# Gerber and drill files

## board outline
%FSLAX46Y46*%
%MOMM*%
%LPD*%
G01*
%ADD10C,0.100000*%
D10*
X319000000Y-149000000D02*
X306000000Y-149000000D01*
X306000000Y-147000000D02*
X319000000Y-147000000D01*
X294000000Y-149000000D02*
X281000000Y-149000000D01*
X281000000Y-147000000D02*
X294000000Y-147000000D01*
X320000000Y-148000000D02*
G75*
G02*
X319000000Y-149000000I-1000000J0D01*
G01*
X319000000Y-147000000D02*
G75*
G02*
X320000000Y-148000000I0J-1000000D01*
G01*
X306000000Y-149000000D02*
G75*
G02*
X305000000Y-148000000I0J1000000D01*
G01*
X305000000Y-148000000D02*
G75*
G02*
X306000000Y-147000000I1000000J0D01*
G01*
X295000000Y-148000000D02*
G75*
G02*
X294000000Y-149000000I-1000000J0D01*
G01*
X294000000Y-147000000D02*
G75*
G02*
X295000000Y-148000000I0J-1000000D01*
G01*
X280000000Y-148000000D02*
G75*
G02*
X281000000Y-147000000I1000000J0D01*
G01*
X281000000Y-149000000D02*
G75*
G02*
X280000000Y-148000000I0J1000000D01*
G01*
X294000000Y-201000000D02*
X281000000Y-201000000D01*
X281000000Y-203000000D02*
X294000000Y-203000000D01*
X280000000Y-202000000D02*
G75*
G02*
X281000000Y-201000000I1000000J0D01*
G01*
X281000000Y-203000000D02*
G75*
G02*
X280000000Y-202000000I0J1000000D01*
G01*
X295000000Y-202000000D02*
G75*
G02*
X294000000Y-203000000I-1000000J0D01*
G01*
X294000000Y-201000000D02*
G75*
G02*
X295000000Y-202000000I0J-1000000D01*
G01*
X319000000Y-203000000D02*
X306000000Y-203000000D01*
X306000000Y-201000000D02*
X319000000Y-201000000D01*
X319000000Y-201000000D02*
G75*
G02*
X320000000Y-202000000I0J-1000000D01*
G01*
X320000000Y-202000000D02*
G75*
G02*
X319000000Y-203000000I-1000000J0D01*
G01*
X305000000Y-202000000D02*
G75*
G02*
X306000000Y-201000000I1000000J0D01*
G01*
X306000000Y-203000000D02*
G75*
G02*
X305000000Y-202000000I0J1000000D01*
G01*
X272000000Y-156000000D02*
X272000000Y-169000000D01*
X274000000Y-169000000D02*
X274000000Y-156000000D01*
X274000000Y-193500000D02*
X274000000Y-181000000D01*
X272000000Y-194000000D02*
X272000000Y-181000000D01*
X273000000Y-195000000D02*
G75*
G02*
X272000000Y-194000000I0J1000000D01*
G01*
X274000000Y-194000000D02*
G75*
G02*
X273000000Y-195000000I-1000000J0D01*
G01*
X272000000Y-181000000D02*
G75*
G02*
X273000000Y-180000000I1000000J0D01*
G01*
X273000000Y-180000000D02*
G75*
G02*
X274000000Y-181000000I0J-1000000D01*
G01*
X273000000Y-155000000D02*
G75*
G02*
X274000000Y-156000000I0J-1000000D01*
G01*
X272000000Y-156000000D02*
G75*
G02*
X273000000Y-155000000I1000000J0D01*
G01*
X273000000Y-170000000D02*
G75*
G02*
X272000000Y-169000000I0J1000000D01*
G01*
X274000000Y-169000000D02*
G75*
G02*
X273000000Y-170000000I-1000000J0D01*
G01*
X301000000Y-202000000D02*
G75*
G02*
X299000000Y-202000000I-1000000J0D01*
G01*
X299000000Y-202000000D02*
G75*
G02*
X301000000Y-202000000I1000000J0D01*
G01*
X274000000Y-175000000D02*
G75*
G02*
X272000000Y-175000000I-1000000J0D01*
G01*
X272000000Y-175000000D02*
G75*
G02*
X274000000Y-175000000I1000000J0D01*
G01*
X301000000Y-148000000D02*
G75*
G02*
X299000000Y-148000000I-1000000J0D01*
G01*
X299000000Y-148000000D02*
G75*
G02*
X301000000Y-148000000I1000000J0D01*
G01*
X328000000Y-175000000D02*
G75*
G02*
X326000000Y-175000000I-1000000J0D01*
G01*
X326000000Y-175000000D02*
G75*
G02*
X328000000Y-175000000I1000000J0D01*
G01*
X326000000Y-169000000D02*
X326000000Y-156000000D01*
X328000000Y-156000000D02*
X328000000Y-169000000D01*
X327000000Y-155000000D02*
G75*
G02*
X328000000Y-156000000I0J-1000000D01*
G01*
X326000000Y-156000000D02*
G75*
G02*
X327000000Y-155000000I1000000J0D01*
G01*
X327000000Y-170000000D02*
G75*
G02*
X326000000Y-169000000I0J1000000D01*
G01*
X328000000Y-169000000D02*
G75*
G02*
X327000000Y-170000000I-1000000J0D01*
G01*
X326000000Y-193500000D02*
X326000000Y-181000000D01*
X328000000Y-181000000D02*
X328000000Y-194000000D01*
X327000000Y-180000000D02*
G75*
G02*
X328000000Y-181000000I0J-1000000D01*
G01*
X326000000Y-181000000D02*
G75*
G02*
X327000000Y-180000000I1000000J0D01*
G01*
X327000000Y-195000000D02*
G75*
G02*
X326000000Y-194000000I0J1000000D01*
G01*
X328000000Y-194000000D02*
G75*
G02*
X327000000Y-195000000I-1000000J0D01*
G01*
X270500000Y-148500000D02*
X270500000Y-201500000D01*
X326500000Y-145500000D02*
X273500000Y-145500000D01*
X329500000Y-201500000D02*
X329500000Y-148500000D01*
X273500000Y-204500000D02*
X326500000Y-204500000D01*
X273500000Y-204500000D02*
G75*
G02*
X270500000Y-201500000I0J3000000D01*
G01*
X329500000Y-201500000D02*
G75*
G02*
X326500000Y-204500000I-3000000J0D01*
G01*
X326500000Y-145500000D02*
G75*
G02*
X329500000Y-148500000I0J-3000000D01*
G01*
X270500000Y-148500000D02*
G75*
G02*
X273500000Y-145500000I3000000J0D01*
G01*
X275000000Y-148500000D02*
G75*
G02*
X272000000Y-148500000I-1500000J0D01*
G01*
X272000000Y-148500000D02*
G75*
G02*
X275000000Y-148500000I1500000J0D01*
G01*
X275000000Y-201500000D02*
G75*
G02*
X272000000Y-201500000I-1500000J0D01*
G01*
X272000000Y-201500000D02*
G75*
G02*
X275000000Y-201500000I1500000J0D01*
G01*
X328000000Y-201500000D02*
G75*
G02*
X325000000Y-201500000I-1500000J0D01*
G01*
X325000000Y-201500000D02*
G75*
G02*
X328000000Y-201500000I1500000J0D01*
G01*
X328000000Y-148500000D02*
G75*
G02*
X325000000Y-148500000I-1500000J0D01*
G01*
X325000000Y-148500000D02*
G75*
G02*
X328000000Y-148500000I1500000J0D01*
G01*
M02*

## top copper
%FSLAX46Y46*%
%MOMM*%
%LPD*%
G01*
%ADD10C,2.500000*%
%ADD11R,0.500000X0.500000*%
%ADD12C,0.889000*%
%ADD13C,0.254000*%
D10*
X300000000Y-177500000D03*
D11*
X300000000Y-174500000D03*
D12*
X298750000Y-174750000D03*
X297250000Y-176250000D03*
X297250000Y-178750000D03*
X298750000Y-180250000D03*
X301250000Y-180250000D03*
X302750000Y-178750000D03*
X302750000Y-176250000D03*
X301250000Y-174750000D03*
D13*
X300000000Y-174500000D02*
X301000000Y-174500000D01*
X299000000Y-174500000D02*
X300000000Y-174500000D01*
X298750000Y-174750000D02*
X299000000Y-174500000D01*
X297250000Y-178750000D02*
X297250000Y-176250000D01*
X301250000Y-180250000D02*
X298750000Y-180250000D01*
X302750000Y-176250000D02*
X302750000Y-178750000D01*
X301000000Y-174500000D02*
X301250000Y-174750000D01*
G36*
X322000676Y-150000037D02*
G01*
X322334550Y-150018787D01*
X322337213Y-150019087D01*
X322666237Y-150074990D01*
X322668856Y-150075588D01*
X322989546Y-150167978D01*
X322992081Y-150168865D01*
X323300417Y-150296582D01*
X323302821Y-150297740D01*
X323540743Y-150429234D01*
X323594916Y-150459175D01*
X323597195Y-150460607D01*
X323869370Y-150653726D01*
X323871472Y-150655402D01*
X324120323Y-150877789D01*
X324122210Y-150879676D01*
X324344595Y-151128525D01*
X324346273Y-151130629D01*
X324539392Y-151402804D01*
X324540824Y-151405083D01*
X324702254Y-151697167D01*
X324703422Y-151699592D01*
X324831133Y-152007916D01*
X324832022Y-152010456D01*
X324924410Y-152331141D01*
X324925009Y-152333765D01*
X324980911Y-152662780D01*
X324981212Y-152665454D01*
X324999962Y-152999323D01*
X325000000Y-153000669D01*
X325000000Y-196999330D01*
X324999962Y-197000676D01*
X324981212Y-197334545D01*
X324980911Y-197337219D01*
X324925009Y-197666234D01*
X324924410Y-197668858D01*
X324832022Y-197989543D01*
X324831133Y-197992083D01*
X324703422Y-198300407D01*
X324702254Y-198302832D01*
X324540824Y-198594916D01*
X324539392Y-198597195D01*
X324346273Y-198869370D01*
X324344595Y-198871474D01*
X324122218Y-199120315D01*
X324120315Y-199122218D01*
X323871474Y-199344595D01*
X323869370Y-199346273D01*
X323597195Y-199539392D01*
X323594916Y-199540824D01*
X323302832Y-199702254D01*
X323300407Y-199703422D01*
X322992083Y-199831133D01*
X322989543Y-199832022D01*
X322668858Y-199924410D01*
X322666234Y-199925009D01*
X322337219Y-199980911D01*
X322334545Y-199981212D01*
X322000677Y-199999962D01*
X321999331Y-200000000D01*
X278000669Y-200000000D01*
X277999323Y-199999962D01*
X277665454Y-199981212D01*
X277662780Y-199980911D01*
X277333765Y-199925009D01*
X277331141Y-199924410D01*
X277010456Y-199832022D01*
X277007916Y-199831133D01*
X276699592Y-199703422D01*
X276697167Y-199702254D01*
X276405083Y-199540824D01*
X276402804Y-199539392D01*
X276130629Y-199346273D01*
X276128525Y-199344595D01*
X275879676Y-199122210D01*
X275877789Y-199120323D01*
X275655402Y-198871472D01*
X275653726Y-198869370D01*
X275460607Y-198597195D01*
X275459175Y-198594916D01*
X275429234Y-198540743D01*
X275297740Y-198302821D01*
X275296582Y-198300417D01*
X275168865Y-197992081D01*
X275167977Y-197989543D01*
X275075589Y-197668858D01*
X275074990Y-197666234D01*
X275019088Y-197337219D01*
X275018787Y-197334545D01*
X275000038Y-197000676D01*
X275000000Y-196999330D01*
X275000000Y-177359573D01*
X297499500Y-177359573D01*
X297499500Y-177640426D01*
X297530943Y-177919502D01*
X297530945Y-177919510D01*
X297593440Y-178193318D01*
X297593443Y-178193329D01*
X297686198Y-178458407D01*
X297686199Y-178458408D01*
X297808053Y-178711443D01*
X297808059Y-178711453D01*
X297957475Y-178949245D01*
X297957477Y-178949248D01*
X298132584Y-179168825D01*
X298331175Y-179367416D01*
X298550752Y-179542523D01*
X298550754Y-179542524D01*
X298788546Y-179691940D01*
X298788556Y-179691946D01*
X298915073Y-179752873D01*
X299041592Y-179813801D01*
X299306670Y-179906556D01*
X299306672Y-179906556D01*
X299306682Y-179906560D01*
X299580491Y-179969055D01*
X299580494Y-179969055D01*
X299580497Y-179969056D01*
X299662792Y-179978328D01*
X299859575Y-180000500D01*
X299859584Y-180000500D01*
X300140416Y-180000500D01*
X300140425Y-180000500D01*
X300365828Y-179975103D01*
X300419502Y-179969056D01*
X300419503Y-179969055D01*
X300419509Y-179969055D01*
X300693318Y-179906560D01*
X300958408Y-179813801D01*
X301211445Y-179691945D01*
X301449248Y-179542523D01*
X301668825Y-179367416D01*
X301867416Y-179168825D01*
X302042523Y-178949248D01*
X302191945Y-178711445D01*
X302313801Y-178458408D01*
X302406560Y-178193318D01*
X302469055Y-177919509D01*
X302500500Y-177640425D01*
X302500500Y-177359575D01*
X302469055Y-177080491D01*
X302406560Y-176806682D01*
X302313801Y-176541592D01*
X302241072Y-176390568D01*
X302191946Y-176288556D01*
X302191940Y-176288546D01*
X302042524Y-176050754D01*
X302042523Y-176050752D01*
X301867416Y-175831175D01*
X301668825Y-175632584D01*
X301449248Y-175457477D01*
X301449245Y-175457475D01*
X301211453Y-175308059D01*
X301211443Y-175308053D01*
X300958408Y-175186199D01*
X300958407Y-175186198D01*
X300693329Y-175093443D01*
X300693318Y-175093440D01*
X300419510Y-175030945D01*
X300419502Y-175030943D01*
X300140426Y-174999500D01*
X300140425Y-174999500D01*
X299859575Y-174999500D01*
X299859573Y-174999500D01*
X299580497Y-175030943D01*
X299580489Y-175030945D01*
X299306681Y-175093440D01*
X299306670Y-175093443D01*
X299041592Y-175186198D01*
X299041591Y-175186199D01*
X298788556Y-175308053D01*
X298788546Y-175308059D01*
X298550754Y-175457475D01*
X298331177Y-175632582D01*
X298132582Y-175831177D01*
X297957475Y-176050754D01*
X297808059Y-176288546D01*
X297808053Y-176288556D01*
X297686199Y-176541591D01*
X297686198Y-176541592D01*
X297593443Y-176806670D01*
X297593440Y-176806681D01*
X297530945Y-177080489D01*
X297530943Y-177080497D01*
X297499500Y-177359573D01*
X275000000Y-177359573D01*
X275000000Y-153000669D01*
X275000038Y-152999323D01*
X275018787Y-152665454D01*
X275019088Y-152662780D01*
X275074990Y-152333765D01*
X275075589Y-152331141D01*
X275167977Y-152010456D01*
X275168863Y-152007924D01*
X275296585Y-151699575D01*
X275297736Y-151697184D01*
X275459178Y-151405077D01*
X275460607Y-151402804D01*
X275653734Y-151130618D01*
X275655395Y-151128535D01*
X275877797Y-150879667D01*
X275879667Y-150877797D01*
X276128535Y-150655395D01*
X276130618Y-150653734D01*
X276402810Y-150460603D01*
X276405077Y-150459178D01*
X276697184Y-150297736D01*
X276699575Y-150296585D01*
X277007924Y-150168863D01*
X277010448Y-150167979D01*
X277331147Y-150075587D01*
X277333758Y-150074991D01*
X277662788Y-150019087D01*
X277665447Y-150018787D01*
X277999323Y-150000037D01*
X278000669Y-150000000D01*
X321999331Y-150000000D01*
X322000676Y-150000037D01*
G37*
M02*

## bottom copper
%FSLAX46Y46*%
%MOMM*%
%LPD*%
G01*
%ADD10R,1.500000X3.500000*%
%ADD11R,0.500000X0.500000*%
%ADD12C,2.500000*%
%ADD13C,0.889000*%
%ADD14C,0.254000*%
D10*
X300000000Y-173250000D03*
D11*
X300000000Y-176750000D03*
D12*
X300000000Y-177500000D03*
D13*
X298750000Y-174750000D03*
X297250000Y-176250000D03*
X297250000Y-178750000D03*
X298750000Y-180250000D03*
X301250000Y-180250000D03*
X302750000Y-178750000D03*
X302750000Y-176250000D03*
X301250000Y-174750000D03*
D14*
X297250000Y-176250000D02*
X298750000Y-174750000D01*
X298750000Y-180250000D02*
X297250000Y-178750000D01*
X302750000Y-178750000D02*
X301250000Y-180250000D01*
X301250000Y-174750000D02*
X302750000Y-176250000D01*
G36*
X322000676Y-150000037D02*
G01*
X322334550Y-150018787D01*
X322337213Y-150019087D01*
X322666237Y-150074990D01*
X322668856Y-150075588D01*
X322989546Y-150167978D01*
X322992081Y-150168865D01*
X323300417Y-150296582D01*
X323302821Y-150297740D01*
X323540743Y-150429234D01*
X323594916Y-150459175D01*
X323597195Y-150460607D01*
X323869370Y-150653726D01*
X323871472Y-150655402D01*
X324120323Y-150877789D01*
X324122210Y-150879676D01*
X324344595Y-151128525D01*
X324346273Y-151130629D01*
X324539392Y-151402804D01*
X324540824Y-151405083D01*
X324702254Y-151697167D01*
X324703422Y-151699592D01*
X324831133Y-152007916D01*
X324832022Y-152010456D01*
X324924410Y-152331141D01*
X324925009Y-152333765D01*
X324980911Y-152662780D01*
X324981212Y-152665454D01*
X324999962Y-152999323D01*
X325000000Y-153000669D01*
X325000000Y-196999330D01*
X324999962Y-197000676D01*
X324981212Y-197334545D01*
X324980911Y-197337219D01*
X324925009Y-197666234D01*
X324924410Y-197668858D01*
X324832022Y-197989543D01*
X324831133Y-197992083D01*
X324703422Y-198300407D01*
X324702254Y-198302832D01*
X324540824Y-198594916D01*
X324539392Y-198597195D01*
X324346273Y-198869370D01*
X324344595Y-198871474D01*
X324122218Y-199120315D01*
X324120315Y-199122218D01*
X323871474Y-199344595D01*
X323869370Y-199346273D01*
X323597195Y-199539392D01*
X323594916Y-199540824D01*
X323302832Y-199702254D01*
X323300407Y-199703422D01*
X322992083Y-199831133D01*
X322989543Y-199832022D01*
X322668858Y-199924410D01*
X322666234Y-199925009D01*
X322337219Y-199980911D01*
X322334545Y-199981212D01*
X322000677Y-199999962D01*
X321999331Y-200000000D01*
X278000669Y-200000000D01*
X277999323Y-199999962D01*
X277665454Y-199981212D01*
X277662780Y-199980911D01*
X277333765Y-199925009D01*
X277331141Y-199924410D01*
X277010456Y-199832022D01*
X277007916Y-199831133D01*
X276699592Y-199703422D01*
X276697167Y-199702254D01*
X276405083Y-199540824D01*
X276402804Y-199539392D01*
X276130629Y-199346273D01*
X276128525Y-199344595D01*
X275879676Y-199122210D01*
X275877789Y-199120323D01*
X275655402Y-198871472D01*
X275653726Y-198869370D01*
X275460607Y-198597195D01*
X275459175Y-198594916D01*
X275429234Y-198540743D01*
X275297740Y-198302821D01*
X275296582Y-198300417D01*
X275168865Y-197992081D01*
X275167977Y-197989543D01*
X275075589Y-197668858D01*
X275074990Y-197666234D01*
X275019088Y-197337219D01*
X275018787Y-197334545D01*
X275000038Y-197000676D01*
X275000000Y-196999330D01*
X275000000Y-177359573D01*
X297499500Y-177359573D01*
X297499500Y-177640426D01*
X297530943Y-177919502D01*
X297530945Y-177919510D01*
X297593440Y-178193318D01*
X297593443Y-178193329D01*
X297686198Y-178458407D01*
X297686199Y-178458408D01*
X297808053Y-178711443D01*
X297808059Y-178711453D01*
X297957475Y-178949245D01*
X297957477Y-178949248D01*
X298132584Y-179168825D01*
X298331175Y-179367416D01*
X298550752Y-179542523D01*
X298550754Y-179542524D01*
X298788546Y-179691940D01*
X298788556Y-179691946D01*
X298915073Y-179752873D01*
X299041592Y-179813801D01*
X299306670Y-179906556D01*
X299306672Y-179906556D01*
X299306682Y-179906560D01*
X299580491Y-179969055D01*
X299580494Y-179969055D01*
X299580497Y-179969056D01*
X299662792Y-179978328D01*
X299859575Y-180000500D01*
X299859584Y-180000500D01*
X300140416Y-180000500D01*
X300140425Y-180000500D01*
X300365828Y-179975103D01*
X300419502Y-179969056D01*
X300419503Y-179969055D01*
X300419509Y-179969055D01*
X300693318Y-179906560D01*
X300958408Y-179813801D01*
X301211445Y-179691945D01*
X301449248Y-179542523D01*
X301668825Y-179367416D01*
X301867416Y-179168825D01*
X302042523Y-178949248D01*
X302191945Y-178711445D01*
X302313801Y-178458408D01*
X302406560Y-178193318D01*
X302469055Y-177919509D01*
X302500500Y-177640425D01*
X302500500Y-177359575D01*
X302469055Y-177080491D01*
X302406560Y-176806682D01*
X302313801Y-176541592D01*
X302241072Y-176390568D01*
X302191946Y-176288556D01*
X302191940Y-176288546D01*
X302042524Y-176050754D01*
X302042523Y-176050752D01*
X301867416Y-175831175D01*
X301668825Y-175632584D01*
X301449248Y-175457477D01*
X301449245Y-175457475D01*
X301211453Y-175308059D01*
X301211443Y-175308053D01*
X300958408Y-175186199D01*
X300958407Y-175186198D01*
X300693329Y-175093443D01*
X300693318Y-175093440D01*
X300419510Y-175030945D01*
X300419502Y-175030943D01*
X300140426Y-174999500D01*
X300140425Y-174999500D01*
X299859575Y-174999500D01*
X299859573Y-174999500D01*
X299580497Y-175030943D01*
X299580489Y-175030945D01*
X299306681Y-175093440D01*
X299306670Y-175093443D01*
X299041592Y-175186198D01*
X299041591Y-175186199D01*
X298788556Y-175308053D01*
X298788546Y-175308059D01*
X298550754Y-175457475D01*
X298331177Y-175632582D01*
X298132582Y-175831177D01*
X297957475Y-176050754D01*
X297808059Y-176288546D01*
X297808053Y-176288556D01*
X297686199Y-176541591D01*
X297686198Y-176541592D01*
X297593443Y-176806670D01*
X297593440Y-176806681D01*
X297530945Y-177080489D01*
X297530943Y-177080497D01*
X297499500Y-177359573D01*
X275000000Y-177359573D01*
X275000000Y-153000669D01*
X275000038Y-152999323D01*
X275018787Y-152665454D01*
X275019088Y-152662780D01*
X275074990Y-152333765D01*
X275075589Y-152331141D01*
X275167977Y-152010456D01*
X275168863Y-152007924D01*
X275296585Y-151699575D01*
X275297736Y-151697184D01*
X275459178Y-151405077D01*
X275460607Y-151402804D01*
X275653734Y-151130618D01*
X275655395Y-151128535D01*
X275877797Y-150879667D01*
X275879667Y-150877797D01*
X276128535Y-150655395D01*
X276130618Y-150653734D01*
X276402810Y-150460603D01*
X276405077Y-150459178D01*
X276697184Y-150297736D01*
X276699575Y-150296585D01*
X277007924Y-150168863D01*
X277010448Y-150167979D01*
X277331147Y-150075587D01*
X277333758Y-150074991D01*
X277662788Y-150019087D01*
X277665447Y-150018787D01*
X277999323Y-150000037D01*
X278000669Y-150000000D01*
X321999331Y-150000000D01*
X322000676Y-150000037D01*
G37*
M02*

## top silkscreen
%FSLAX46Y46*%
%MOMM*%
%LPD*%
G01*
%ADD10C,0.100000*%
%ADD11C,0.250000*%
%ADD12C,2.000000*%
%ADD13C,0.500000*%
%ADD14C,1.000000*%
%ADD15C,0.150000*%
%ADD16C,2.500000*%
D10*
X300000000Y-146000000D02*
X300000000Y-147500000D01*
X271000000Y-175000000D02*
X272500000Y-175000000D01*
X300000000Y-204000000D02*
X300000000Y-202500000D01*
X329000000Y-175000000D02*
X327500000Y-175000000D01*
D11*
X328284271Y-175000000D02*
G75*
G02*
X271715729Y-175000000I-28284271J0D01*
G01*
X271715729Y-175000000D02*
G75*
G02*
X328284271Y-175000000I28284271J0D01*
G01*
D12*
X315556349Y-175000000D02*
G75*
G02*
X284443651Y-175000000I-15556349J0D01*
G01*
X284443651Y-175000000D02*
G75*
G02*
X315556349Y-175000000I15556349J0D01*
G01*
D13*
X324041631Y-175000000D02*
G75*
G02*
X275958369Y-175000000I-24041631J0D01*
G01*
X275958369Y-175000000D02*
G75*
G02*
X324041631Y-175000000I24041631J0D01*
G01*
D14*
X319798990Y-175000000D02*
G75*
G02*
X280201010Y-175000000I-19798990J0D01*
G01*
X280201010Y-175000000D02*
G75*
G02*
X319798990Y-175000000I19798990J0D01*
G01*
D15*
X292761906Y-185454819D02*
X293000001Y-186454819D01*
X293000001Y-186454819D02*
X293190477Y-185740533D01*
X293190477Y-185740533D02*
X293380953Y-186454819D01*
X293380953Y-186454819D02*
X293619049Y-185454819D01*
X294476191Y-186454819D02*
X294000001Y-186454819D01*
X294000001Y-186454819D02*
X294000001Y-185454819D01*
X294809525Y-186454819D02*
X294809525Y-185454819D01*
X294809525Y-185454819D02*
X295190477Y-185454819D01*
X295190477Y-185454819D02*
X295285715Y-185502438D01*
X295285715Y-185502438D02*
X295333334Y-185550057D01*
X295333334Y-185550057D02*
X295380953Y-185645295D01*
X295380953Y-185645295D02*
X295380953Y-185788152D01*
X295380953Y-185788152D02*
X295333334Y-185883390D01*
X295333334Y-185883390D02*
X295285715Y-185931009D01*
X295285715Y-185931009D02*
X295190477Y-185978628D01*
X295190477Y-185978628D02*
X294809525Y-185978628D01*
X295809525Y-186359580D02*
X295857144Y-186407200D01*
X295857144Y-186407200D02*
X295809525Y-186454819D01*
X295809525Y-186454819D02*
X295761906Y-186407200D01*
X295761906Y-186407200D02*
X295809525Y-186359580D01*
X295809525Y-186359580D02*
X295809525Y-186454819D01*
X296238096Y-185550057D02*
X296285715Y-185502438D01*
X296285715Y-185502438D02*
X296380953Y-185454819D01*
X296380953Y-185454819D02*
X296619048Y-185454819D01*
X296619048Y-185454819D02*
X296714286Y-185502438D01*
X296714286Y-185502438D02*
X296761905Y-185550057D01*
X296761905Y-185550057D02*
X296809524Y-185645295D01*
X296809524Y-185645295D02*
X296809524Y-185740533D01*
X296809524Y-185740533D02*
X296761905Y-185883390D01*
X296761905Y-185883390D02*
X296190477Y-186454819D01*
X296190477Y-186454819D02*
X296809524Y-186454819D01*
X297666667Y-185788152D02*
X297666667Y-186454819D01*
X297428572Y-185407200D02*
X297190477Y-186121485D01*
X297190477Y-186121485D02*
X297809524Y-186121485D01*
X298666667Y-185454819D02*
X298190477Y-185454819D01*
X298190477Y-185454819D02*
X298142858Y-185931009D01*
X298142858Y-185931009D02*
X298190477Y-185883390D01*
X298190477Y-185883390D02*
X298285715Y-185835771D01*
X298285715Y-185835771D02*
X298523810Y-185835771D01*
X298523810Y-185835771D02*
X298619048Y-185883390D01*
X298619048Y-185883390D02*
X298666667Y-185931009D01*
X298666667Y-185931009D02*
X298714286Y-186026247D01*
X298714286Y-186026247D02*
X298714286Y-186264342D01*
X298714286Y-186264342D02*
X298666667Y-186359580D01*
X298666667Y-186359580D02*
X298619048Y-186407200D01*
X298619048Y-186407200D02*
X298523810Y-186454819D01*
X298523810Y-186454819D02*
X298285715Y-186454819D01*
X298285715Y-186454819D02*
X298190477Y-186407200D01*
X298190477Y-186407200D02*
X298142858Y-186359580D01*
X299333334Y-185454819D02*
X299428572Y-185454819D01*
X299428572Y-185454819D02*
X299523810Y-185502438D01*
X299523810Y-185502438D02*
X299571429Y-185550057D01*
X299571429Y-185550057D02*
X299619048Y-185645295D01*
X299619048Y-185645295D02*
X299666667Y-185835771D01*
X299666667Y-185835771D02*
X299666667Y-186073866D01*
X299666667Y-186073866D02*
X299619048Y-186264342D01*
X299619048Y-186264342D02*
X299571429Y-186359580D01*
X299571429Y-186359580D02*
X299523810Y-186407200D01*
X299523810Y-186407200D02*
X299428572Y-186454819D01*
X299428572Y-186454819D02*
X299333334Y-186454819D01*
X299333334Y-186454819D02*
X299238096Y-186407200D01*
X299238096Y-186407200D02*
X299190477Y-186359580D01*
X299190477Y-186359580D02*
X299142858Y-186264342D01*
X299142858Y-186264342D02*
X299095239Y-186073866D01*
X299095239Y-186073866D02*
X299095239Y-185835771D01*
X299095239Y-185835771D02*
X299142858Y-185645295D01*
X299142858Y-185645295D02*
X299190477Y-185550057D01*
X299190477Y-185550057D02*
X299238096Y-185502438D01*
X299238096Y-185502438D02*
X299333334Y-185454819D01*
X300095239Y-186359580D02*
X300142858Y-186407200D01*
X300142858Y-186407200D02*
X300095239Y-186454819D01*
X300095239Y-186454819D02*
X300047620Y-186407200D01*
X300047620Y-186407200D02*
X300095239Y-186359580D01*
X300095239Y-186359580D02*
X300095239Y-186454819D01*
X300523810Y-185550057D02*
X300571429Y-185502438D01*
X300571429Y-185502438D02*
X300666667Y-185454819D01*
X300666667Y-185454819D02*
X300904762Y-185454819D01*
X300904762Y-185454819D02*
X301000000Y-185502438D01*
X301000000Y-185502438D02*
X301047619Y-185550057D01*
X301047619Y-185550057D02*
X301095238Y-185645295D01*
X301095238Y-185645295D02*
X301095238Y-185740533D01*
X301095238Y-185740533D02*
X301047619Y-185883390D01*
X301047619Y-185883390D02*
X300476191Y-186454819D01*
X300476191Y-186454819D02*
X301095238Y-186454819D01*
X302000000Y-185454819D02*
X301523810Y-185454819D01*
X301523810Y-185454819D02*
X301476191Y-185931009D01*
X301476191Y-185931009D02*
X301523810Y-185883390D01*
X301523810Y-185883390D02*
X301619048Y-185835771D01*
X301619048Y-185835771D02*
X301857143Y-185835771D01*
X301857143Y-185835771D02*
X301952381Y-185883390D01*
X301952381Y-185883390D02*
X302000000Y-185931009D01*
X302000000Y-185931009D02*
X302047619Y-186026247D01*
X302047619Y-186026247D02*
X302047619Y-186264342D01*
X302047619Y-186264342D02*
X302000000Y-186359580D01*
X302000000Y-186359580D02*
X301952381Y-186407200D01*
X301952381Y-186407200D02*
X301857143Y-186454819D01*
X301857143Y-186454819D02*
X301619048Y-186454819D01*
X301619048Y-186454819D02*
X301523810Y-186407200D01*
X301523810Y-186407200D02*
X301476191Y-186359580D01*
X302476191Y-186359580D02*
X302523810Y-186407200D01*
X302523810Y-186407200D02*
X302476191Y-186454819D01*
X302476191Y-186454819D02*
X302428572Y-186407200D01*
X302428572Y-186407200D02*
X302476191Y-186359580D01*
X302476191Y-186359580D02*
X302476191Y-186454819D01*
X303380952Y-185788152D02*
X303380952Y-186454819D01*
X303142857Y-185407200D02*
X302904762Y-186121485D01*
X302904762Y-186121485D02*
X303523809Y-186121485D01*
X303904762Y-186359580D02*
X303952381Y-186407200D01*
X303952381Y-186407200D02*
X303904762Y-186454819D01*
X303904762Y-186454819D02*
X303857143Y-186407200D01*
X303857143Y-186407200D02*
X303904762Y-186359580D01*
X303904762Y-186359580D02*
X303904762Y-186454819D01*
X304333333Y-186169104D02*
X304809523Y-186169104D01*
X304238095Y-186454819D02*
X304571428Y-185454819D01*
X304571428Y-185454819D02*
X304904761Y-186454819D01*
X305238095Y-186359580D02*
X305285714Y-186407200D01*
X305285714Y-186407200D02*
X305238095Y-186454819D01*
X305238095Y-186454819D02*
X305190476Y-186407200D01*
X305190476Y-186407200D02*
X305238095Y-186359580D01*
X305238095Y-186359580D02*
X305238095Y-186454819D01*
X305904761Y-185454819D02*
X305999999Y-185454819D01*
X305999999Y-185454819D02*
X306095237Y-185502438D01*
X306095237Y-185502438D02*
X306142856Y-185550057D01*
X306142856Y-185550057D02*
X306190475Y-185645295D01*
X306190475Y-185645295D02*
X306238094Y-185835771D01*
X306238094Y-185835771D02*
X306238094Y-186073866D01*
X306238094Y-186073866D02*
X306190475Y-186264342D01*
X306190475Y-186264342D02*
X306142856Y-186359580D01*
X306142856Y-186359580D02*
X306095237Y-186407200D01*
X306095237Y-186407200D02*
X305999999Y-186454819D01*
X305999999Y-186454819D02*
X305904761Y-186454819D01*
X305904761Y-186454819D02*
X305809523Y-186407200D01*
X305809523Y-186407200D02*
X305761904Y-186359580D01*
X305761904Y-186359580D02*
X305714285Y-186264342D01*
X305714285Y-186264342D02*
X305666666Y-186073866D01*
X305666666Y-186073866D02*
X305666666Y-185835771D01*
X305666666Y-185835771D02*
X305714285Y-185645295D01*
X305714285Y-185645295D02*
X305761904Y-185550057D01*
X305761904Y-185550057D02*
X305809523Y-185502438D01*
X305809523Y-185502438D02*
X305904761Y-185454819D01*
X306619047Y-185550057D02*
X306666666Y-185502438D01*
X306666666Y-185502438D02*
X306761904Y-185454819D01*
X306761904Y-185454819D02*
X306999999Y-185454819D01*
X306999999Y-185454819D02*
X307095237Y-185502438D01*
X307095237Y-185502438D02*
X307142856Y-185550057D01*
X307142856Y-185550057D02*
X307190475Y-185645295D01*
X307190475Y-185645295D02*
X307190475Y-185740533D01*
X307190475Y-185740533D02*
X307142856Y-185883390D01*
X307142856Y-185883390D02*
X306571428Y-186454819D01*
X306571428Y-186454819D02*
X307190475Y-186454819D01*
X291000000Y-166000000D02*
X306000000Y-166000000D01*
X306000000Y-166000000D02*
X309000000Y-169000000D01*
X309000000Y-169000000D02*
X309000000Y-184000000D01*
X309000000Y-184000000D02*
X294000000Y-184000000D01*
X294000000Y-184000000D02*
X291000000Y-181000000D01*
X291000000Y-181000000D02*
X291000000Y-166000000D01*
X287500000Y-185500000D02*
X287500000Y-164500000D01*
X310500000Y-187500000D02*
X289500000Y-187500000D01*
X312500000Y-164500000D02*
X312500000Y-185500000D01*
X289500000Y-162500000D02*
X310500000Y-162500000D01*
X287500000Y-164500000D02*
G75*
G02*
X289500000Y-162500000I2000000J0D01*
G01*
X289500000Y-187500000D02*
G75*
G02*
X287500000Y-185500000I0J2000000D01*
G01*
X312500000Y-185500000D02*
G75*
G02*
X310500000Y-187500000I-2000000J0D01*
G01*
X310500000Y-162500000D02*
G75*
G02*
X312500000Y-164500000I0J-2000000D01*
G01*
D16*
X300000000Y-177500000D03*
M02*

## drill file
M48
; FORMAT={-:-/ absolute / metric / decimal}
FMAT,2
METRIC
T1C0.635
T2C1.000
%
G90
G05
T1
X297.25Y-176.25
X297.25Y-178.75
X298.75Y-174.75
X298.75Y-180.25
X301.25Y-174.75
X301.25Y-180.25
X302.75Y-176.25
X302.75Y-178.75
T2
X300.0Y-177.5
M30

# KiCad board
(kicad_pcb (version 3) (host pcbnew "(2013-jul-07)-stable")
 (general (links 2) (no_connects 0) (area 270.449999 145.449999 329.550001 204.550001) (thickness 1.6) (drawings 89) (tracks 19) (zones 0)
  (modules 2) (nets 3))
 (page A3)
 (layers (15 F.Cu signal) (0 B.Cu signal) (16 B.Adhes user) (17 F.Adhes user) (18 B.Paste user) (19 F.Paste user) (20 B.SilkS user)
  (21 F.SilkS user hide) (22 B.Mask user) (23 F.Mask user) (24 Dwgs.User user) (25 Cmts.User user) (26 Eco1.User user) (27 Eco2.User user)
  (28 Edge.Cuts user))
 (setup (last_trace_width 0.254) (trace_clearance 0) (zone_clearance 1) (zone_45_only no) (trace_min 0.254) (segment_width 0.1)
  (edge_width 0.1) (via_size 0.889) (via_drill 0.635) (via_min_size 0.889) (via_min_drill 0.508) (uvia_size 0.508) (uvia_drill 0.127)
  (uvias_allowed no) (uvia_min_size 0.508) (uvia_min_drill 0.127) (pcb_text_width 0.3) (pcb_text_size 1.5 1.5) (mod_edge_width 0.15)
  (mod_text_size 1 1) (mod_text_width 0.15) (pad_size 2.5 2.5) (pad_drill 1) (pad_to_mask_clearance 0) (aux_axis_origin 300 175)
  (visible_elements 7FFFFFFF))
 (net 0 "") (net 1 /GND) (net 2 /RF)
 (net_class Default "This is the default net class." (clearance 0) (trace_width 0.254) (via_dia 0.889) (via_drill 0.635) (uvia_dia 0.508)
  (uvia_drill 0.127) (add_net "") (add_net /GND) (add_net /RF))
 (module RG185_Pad (layer B.Cu) (at 300 175.75 270)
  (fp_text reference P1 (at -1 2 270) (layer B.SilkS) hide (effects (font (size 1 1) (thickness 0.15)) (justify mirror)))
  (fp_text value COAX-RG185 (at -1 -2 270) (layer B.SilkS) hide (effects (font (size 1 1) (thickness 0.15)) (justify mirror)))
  (pad 1 connect rect (at -2.5 0 270) (size 3.5 1.5) (layers B.Cu B.Mask) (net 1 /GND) (die_length 1))
  (pad 2 connect rect (at 1 0 270) (size 0.5 0.5) (layers B.Cu B.Mask) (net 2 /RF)))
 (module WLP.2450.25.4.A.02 (layer F.Cu) (at 300 175)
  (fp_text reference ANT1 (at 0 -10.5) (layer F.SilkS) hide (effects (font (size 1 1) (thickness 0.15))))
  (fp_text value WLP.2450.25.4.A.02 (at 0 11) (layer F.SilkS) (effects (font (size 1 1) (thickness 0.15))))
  (fp_line (start -9 -9) (end 6 -9) (layer F.SilkS) (width 0.15))
  (fp_line (start 6 -9) (end 9 -6) (layer F.SilkS) (width 0.15))
  (fp_line (start 9 -6) (end 9 9) (layer F.SilkS) (width 0.15))
  (fp_line (start 9 9) (end -6 9) (layer F.SilkS) (width 0.15))
  (fp_line (start -6 9) (end -9 6) (layer F.SilkS) (width 0.15))
  (fp_line (start -9 6) (end -9 -9) (layer F.SilkS) (width 0.15))
  (fp_line (start -12.5 10.5) (end -12.5 -10.5) (layer F.SilkS) (width 0.15))
  (fp_line (start 10.5 12.5) (end -10.5 12.5) (layer F.SilkS) (width 0.15))
  (fp_line (start 12.5 -10.5) (end 12.5 10.5) (layer F.SilkS) (width 0.15))
  (fp_line (start -10.5 -12.5) (end 10.5 -12.5) (layer F.SilkS) (width 0.15))
  (fp_arc (start -10.5 -10.5) (end -12.5 -10.5) (angle 90) (layer F.SilkS) (width 0.15))
  (fp_arc (start -10.5 10.5) (end -10.5 12.5) (angle 90) (layer F.SilkS) (width 0.15))
  (fp_arc (start 10.5 10.5) (end 12.5 10.5) (angle 90) (layer F.SilkS) (width 0.15))
  (fp_arc (start 10.5 -10.5) (end 10.5 -12.5) (angle 90) (layer F.SilkS) (width 0.15))
  (pad 2 thru_hole circle (at 0 2.5) (size 2.5 2.5) (drill 1) (layers *.Mask B.Cu F.SilkS) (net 2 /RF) (clearance 1.25))
  (pad 1 connect rect (at 0 -0.5) (size 0.5 0.5) (layers F.Cu) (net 1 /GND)))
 (gr_line (start 319 149) (end 306 149) (angle 90) (layer Edge.Cuts) (width 0.1))
 (gr_line (start 306 147) (end 319 147) (angle 90) (layer Edge.Cuts) (width 0.1))
 (gr_line (start 294 149) (end 281 149) (angle 90) (layer Edge.Cuts) (width 0.1))
 (gr_line (start 281 147) (end 294 147) (angle 90) (layer Edge.Cuts) (width 0.1))
 (gr_arc (start 319 148) (end 320 148) (angle 90) (layer Edge.Cuts) (width 0.1))
 (gr_arc (start 319 148) (end 319 147) (angle 90) (layer Edge.Cuts) (width 0.1))
 (gr_arc (start 306 148) (end 306 149) (angle 90) (layer Edge.Cuts) (width 0.1))
 (gr_arc (start 306 148) (end 305 148) (angle 90) (layer Edge.Cuts) (width 0.1))
 (gr_arc (start 294 148) (end 295 148) (angle 90) (layer Edge.Cuts) (width 0.1))
 (gr_arc (start 294 148) (end 294 147) (angle 90) (layer Edge.Cuts) (width 0.1))
 (gr_arc (start 281 148) (end 280 148) (angle 90) (layer Edge.Cuts) (width 0.1))
 (gr_arc (start 281 148) (end 281 149) (angle 90) (layer Edge.Cuts) (width 0.1))
 (gr_line (start 294 201) (end 281 201) (angle 90) (layer Edge.Cuts) (width 0.1))
 (gr_line (start 281 203) (end 294 203) (angle 90) (layer Edge.Cuts) (width 0.1))
 (gr_arc (start 281 202) (end 280 202) (angle 90) (layer Edge.Cuts) (width 0.1))
 (gr_arc (start 281 202) (end 281 203) (angle 90) (layer Edge.Cuts) (width 0.1))
 (gr_arc (start 294 202) (end 295 202) (angle 90) (layer Edge.Cuts) (width 0.1))
 (gr_arc (start 294 202) (end 294 201) (angle 90) (layer Edge.Cuts) (width 0.1))
 (gr_line (start 319 203) (end 306 203) (angle 90) (layer Edge.Cuts) (width 0.1))
 (gr_line (start 306 201) (end 319 201) (angle 90) (layer Edge.Cuts) (width 0.1))
 (gr_arc (start 319 202) (end 319 201) (angle 90) (layer Edge.Cuts) (width 0.1))
 (gr_arc (start 319 202) (end 320 202) (angle 90) (layer Edge.Cuts) (width 0.1))
 (gr_arc (start 306 202) (end 305 202) (angle 90) (layer Edge.Cuts) (width 0.1))
 (gr_arc (start 306 202) (end 306 203) (angle 90) (layer Edge.Cuts) (width 0.1))
 (gr_line (start 272 156) (end 272 169) (angle 90) (layer Edge.Cuts) (width 0.1))
 (gr_line (start 274 169) (end 274 156) (angle 90) (layer Edge.Cuts) (width 0.1))
 (gr_line (start 274 193.5) (end 274 181) (angle 90) (layer Edge.Cuts) (width 0.1))
 (gr_line (start 272 194) (end 272 181) (angle 90) (layer Edge.Cuts) (width 0.1))
 (gr_arc (start 273 194) (end 273 195) (angle 90) (layer Edge.Cuts) (width 0.1))
 (gr_arc (start 273 194) (end 274 194) (angle 90) (layer Edge.Cuts) (width 0.1))
 (gr_arc (start 273 181) (end 272 181) (angle 90) (layer Edge.Cuts) (width 0.1))
 (gr_arc (start 273 181) (end 273 180) (angle 90) (layer Edge.Cuts) (width 0.1))
 (gr_arc (start 273 156) (end 273 155) (angle 90) (layer Edge.Cuts) (width 0.1))
 (gr_arc (start 273 156) (end 272 156) (angle 90) (layer Edge.Cuts) (width 0.1))
 (gr_arc (start 273 169) (end 273 170) (angle 90) (layer Edge.Cuts) (width 0.1))
 (gr_arc (start 273 169) (end 274 169) (angle 90) (layer Edge.Cuts) (width 0.1))
 (gr_circle (center 300 202) (end 300 203) (layer Edge.Cuts) (width 0.1))
 (gr_circle (center 273 175) (end 272 175) (layer Edge.Cuts) (width 0.1))
 (gr_circle (center 300 148) (end 300 147) (layer Edge.Cuts) (width 0.1))
 (gr_circle (center 327 175) (end 327 174) (layer Edge.Cuts) (width 0.1))
 (gr_line (start 326 169) (end 326 156) (angle 90) (layer Edge.Cuts) (width 0.1))
 (gr_line (start 328 156) (end 328 169) (angle 90) (layer Edge.Cuts) (width 0.1))
 (gr_arc (start 327 156) (end 327 155) (angle 90) (layer Edge.Cuts) (width 0.1))
 (gr_arc (start 327 156) (end 326 156) (angle 90) (layer Edge.Cuts) (width 0.1))
 (gr_arc (start 327 169) (end 327 170) (angle 90) (layer Edge.Cuts) (width 0.1))
 (gr_arc (start 327 169) (end 328 169) (angle 90) (layer Edge.Cuts) (width 0.1))
 (gr_line (start 326 193.5) (end 326 181) (angle 90) (layer Edge.Cuts) (width 0.1))
 (gr_line (start 328 181) (end 328 194) (angle 90) (layer Edge.Cuts) (width 0.1))
 (gr_arc (start 327 181) (end 327 180) (angle 90) (layer Edge.Cuts) (width 0.1))
 (gr_arc (start 327 181) (end 326 181) (angle 90) (layer Edge.Cuts) (width 0.1))
 (gr_arc (start 327 194) (end 327 195) (angle 90) (layer Edge.Cuts) (width 0.1))
 (gr_arc (start 327 194) (end 328 194) (angle 90) (layer Edge.Cuts) (width 0.1))
 (gr_line (start 300 146) (end 300 147.5) (angle 90) (layer F.SilkS) (width 0.1))
 (gr_line (start 271 175) (end 272.5 175) (angle 90) (layer F.SilkS) (width 0.1))
 (gr_line (start 300 204) (end 300 202.5) (angle 90) (layer F.SilkS) (width 0.1))
 (gr_line (start 329 175) (end 327.5 175) (angle 90) (layer F.SilkS) (width 0.1))
 (gr_arc (start 300 175) (end 320 155) (angle 360) (layer F.SilkS) (width 0.25))
 (gr_arc (start 300 175) (end 311 164) (angle 360) (layer F.SilkS) (width 2))
 (gr_arc (start 300 175) (end 317 158) (angle 360) (layer F.SilkS) (width 0.5))
 (gr_arc (start 300 175) (end 314 161) (angle 360) (layer F.SilkS) (width 1))
 (gr_line (start 270.5 148.5) (end 270.5 201.5) (angle 90) (layer Edge.Cuts) (width 0.1))
 (gr_line (start 326.5 145.5) (end 273.5 145.5) (angle 90) (layer Edge.Cuts) (width 0.1))
 (gr_line (start 329.5 201.5) (end 329.5 148.5) (angle 90) (layer Edge.Cuts) (width 0.1))
 (gr_line (start 273.5 204.5) (end 326.5 204.5) (angle 90) (layer Edge.Cuts) (width 0.1))
 (gr_arc (start 273.5 201.5) (end 273.5 204.5) (angle 90) (layer Edge.Cuts) (width 0.1))
 (gr_arc (start 326.5 201.5) (end 329.5 201.5) (angle 90) (layer Edge.Cuts) (width 0.1))
 (gr_arc (start 326.5 148.5) (end 326.5 145.5) (angle 90) (layer Edge.Cuts) (width 0.1))
 (gr_arc (start 273.5 148.5) (end 270.5 148.5) (angle 90) (layer Edge.Cuts) (width 0.1))
 (gr_circle (center 273.5 148.5) (end 275 148.5) (layer Edge.Cuts) (width 0.1))
 (gr_circle (center 273.5 201.5) (end 273.5 200) (layer Edge.Cuts) (width 0.1))
 (gr_circle (center 326.5 201.5) (end 326.5 200) (layer Edge.Cuts) (width 0.1))
 (gr_circle (center 326.5 148.5) (end 325 148.5) (layer Edge.Cuts) (width 0.1))
 (segment (start 300 174.5) (end 301 174.5) (width 0.254) (layer F.Cu) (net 1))
 (segment (start 299 174.5) (end 300 174.5) (width 0.254) (layer F.Cu) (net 1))
 (segment (start 298.75 174.75) (end 299 174.5) (width 0.254) (layer F.Cu) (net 1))
 (via blind (at 298.75 174.75) (size 0.889) (layers F.Cu B.Cu) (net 1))
 (segment (start 297.25 176.25) (end 298.75 174.75) (width 0.254) (layer B.Cu) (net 1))
 (via blind (at 297.25 176.25) (size 0.889) (layers F.Cu B.Cu) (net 1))
 (segment (start 297.25 178.75) (end 297.25 176.25) (width 0.254) (layer F.Cu) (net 1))
 (via blind (at 297.25 178.75) (size 0.889) (layers F.Cu B.Cu) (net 1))
 (segment (start 298.75 180.25) (end 297.25 178.75) (width 0.254) (layer B.Cu) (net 1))
 (via blind (at 298.75 180.25) (size 0.889) (layers F.Cu B.Cu) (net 1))
 (segment (start 301.25 180.25) (end 298.75 180.25) (width 0.254) (layer F.Cu) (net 1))
 (via blind (at 301.25 180.25) (size 0.889) (layers F.Cu B.Cu) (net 1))
 (segment (start 302.75 178.75) (end 301.25 180.25) (width 0.254) (layer B.Cu) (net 1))
 (via blind (at 302.75 178.75) (size 0.889) (layers F.Cu B.Cu) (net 1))
 (segment (start 302.75 176.25) (end 302.75 178.75) (width 0.254) (layer F.Cu) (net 1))
 (via blind (at 302.75 176.25) (size 0.889) (layers F.Cu B.Cu) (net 1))
 (segment (start 301.25 174.75) (end 302.75 176.25) (width 0.254) (layer B.Cu) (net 1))
 (via blind (at 301.25 174.75) (size 0.889) (layers F.Cu B.Cu) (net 1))
 (segment (start 301 174.5) (end 301.25 174.75) (width 0.254) (layer F.Cu) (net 1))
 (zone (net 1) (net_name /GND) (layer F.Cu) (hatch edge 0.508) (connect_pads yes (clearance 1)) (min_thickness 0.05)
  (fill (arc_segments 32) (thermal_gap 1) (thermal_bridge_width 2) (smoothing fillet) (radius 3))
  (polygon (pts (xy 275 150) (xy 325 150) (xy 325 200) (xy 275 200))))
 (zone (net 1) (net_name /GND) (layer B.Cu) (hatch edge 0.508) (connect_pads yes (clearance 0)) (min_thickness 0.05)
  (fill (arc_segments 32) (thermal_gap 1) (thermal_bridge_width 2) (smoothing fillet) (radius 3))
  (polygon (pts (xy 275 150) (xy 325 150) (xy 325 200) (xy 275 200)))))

